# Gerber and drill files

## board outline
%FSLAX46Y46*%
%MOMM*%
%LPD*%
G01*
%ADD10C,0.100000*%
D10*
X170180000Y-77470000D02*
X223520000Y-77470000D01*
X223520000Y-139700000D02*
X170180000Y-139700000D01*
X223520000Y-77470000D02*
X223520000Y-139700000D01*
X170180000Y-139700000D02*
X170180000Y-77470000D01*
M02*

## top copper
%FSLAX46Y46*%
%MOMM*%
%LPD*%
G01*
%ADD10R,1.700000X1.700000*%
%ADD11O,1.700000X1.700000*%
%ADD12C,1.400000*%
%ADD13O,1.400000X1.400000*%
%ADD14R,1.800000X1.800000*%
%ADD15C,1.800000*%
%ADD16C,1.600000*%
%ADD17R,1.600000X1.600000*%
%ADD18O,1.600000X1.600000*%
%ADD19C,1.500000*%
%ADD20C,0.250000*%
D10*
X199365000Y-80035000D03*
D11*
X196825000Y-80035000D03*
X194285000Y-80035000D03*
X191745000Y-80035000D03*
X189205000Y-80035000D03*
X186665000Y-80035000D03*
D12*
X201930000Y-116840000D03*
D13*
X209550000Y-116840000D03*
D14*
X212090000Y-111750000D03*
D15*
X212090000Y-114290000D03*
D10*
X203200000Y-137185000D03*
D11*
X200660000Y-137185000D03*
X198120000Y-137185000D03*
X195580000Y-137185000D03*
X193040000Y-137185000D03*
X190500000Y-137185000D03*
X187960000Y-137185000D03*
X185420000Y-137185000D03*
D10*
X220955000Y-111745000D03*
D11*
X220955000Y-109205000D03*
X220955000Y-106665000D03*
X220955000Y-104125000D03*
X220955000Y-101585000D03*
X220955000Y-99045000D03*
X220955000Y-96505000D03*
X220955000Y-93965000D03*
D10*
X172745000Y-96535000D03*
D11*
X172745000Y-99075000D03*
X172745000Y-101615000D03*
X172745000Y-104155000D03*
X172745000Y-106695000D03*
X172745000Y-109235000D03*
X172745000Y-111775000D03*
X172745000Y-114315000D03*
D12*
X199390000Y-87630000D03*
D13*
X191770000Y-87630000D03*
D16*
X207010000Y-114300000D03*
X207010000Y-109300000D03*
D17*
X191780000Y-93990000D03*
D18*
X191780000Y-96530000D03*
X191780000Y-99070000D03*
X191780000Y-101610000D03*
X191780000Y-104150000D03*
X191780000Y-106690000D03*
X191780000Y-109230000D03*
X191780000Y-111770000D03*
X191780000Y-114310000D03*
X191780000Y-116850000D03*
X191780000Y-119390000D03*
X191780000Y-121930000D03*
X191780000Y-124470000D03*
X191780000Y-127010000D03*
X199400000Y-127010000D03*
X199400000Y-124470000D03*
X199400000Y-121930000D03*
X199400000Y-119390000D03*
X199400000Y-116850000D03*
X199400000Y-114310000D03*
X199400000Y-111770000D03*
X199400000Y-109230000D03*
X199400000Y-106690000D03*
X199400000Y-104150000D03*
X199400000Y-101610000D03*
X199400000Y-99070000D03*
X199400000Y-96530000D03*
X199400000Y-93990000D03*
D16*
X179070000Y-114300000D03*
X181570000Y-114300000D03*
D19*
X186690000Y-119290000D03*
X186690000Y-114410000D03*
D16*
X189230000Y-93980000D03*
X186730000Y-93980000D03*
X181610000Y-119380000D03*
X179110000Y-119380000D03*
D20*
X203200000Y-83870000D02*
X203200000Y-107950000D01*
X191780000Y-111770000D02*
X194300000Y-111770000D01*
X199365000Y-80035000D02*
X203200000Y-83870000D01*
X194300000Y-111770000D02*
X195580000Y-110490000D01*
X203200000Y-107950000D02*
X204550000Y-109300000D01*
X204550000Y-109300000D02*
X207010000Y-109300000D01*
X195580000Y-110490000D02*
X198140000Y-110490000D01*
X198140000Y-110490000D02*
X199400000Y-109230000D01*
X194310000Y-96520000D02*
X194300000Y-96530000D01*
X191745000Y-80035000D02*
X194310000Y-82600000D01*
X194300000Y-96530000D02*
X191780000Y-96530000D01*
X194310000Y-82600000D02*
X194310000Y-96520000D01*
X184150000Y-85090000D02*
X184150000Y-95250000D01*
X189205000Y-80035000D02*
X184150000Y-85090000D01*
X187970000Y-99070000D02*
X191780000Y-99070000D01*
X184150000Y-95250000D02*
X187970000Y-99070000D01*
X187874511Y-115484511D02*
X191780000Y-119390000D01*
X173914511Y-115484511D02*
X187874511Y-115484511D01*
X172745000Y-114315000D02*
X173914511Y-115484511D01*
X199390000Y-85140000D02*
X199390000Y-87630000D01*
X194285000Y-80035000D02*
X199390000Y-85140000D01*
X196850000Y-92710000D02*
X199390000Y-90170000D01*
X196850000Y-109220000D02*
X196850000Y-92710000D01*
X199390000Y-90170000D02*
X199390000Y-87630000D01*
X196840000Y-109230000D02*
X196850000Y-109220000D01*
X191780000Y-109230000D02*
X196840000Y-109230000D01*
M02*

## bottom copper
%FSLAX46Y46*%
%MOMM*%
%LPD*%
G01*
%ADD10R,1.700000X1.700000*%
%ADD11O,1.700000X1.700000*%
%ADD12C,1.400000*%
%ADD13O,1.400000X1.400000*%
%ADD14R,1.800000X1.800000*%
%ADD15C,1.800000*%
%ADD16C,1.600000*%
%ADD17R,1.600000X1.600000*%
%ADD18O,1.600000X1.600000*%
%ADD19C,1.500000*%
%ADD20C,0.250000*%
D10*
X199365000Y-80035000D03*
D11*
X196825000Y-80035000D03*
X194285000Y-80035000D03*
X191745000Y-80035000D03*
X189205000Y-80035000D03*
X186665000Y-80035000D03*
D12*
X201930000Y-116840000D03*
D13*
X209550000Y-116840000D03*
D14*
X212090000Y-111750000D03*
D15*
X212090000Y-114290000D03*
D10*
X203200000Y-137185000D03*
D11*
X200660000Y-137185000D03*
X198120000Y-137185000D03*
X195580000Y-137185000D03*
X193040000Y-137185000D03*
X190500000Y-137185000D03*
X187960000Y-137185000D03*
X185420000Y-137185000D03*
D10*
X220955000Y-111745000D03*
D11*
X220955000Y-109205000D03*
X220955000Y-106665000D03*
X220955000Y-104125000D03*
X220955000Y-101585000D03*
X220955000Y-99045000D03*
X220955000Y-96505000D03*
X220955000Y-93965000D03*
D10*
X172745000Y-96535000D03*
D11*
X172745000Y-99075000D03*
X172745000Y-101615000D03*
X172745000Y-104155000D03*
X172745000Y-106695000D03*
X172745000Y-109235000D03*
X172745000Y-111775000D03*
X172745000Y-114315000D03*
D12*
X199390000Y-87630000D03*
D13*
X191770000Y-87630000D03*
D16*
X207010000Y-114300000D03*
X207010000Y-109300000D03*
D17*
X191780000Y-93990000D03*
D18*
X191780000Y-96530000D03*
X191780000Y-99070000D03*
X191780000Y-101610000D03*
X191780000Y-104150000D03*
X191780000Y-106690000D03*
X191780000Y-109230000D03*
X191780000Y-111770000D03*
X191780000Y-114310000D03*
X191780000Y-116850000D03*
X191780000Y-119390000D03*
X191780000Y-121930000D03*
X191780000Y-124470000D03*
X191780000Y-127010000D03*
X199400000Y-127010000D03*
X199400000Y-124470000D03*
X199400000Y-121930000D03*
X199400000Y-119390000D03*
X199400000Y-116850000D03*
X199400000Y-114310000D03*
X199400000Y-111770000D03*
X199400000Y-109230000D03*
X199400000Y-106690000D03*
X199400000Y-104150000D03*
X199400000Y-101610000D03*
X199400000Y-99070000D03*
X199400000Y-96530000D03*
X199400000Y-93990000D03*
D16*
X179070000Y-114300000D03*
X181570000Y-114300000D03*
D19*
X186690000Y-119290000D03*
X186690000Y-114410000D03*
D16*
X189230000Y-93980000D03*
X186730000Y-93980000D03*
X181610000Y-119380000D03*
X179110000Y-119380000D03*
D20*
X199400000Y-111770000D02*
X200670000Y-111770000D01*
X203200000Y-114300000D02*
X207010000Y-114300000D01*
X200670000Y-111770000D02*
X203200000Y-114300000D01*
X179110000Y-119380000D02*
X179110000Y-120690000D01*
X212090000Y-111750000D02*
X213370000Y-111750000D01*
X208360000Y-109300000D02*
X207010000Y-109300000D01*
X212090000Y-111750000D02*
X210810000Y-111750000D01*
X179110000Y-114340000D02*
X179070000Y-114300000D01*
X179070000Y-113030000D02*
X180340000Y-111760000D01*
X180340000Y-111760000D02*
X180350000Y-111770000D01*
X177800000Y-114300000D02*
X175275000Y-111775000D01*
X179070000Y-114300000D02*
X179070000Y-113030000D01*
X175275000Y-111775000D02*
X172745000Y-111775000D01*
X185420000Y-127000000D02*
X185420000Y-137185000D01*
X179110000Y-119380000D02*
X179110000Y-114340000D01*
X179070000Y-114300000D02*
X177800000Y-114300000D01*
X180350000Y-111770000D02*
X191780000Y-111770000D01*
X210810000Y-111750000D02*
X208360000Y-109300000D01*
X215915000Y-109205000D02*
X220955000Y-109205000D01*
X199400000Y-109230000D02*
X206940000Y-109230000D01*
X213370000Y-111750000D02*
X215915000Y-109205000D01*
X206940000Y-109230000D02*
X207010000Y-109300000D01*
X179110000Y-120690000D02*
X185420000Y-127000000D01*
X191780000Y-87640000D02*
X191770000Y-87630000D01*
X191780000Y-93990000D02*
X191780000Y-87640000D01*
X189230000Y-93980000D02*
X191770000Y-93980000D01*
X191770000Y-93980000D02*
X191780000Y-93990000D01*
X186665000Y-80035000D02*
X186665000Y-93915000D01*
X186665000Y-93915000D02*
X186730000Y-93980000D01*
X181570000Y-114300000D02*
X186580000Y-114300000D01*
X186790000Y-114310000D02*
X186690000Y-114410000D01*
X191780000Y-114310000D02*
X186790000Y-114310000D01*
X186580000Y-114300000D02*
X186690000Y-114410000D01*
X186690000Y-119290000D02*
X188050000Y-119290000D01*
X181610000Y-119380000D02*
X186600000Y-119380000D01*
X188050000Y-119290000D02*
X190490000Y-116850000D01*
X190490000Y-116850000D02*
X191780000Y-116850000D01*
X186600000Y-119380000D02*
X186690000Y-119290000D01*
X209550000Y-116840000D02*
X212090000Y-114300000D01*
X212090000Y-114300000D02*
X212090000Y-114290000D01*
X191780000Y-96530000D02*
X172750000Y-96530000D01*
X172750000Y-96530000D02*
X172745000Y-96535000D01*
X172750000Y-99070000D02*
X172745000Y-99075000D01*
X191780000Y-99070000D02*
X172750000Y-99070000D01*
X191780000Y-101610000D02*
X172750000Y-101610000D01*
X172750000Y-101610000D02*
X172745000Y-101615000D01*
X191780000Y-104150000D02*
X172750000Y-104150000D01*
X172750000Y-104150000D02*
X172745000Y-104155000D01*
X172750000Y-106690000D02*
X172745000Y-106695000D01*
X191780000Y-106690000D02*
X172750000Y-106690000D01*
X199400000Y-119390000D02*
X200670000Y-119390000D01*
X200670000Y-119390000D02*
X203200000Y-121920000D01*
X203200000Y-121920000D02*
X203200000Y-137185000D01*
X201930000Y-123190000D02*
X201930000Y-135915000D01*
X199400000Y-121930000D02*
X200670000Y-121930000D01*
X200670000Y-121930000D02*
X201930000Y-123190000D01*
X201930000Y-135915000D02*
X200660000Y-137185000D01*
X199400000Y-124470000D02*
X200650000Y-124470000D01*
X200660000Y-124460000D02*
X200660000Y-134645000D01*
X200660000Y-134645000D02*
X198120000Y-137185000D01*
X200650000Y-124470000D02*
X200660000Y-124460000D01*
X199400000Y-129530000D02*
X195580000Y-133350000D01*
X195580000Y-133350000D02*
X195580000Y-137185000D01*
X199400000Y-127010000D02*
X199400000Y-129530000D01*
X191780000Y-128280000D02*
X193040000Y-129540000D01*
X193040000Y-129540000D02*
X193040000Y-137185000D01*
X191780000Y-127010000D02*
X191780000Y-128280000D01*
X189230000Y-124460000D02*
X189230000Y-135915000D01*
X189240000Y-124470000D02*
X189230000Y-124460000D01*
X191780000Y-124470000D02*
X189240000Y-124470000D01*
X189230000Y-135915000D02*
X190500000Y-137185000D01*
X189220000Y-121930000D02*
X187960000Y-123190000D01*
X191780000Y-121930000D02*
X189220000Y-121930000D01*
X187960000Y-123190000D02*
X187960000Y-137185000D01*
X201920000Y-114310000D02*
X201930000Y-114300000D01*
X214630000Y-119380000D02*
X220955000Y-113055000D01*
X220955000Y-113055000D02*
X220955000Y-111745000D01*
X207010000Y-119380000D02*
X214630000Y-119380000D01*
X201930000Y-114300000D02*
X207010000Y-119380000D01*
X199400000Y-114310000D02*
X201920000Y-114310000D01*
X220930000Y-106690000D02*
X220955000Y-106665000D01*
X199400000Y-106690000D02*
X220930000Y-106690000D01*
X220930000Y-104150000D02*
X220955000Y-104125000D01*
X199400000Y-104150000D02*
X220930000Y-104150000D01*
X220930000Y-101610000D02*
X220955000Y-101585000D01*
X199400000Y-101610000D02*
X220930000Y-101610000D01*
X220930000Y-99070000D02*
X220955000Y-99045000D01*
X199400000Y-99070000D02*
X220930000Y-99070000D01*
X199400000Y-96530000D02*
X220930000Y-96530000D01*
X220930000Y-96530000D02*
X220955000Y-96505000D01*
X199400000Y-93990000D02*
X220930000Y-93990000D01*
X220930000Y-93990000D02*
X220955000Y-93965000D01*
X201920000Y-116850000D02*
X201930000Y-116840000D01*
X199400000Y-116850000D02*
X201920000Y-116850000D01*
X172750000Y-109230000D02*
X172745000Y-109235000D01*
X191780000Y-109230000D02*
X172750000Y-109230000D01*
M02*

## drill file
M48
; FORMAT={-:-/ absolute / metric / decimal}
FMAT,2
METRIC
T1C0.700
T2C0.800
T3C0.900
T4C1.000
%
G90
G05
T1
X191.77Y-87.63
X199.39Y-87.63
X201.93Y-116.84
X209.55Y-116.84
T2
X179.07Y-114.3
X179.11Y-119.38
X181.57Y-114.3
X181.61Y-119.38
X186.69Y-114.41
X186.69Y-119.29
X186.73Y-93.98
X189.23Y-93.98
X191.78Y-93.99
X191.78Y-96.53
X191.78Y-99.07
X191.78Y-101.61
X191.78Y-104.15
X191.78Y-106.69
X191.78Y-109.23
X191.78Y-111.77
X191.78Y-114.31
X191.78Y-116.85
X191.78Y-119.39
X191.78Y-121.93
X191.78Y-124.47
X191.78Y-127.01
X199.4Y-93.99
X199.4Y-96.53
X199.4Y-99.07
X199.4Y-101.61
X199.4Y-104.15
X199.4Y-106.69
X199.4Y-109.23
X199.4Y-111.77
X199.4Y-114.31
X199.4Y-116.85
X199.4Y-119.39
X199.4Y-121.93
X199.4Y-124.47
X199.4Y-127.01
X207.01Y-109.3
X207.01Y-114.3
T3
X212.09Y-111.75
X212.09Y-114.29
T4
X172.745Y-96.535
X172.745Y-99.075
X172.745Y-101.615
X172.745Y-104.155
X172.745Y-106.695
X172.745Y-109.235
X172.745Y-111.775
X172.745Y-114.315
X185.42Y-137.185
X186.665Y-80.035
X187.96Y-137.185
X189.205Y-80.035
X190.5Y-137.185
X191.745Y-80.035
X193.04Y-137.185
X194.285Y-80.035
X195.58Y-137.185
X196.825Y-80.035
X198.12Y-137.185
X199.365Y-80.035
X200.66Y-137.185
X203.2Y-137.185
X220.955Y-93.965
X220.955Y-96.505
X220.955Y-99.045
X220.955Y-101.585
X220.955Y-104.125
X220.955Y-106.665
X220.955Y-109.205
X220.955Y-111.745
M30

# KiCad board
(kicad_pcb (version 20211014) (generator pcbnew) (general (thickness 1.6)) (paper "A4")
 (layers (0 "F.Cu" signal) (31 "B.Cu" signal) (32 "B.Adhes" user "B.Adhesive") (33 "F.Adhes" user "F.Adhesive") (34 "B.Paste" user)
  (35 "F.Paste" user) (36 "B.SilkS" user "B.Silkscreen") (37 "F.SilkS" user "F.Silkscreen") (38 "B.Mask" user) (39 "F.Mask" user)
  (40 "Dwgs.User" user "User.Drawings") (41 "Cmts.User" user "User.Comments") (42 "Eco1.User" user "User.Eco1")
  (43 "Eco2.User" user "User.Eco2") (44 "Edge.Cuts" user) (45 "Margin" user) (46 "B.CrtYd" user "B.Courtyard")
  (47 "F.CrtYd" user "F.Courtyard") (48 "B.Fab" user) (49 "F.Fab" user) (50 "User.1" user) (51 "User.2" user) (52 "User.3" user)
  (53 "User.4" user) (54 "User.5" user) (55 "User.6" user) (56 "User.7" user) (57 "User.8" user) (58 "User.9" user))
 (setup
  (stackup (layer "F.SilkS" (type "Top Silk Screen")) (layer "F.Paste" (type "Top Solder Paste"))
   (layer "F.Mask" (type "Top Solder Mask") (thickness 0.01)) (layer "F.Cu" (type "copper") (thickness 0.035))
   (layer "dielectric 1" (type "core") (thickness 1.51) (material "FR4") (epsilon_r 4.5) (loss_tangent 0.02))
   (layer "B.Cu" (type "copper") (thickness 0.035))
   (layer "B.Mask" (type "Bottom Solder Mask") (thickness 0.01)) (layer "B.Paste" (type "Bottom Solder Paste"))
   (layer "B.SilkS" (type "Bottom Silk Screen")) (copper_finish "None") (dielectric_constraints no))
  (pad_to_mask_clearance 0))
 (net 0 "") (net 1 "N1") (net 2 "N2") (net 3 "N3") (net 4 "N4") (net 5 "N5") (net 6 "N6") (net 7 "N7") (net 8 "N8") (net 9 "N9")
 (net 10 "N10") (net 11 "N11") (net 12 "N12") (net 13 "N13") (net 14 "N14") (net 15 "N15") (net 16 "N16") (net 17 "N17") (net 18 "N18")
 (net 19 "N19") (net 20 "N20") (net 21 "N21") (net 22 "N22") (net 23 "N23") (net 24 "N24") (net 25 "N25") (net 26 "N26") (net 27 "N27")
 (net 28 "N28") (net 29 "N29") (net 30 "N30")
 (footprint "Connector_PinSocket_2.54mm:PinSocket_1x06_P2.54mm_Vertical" (layer "F.Cu") (at 199.365 80.035 -90)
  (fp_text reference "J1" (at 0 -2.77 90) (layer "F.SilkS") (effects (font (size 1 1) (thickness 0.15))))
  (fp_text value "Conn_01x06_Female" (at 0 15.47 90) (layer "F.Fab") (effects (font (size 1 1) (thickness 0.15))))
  (pad "1" thru_hole rect locked (at 0 0 270) (size 1.7 1.7) (drill 1) (layers *.Cu *.Mask) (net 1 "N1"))
  (pad "2" thru_hole oval locked (at 0 2.54 270) (size 1.7 1.7) (drill 1) (layers *.Cu *.Mask) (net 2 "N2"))
  (pad "3" thru_hole oval locked (at 0 5.08 270) (size 1.7 1.7) (drill 1) (layers *.Cu *.Mask) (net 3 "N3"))
  (pad "4" thru_hole oval locked (at 0 7.62 270) (size 1.7 1.7) (drill 1) (layers *.Cu *.Mask) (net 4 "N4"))
  (pad "5" thru_hole oval locked (at 0 10.16 270) (size 1.7 1.7) (drill 1) (layers *.Cu *.Mask) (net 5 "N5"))
  (pad "6" thru_hole oval locked (at 0 12.7 270) (size 1.7 1.7) (drill 1) (layers *.Cu *.Mask) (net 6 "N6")))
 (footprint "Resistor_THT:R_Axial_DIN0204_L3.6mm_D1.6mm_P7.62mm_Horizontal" (layer "F.Cu") (at 201.93 116.84)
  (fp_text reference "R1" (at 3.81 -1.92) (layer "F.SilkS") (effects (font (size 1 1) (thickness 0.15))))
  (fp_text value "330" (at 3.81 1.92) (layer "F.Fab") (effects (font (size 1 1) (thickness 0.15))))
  (pad "1" thru_hole circle locked (at 0 0) (size 1.4 1.4) (drill 0.7) (layers *.Cu *.Mask) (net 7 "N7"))
  (pad "2" thru_hole oval locked (at 7.62 0) (size 1.4 1.4) (drill 0.7) (layers *.Cu *.Mask) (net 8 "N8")))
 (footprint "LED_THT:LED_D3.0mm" (layer "F.Cu") (at 212.09 111.75 -90)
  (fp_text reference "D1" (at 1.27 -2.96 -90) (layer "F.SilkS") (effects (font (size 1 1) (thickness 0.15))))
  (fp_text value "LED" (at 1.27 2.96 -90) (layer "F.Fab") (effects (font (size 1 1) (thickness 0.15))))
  (pad "1" thru_hole rect locked (at 0 0 270) (size 1.8 1.8) (drill 0.9) (layers *.Cu *.Mask) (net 1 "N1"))
  (pad "2" thru_hole circle locked (at 2.54 0 270) (size 1.8 1.8) (drill 0.9) (layers *.Cu *.Mask) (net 8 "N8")))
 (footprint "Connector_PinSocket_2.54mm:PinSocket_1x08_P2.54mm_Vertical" (layer "F.Cu") (at 203.2 137.185 -90)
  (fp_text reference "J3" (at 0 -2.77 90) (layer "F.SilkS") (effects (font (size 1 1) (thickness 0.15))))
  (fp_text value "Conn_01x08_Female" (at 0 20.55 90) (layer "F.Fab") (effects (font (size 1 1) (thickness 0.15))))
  (pad "1" thru_hole rect locked (at 0 0 270) (size 1.7 1.7) (drill 1) (layers *.Cu *.Mask) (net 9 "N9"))
  (pad "2" thru_hole oval locked (at 0 2.54 270) (size 1.7 1.7) (drill 1) (layers *.Cu *.Mask) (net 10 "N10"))
  (pad "3" thru_hole oval locked (at 0 5.08 270) (size 1.7 1.7) (drill 1) (layers *.Cu *.Mask) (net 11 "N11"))
  (pad "4" thru_hole oval locked (at 0 7.62 270) (size 1.7 1.7) (drill 1) (layers *.Cu *.Mask) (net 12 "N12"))
  (pad "5" thru_hole oval locked (at 0 10.16 270) (size 1.7 1.7) (drill 1) (layers *.Cu *.Mask) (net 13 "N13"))
  (pad "6" thru_hole oval locked (at 0 12.7 270) (size 1.7 1.7) (drill 1) (layers *.Cu *.Mask) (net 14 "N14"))
  (pad "7" thru_hole oval locked (at 0 15.24 270) (size 1.7 1.7) (drill 1) (layers *.Cu *.Mask) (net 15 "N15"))
  (pad "8" thru_hole oval locked (at 0 17.78 270) (size 1.7 1.7) (drill 1) (layers *.Cu *.Mask) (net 1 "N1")))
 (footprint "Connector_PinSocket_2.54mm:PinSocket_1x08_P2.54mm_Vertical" (layer "F.Cu") (at 220.955 111.745 180)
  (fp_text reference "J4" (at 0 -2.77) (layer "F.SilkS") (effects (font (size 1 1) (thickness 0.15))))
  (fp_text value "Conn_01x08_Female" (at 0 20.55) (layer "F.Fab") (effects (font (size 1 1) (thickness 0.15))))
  (pad "1" thru_hole rect locked (at 0 0 180) (size 1.7 1.7) (drill 1) (layers *.Cu *.Mask) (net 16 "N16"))
  (pad "2" thru_hole oval locked (at 0 2.54 180) (size 1.7 1.7) (drill 1) (layers *.Cu *.Mask) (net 1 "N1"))
  (pad "3" thru_hole oval locked (at 0 5.08 180) (size 1.7 1.7) (drill 1) (layers *.Cu *.Mask) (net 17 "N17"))
  (pad "4" thru_hole oval locked (at 0 7.62 180) (size 1.7 1.7) (drill 1) (layers *.Cu *.Mask) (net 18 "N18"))
  (pad "5" thru_hole oval locked (at 0 10.16 180) (size 1.7 1.7) (drill 1) (layers *.Cu *.Mask) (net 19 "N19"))
  (pad "6" thru_hole oval locked (at 0 12.7 180) (size 1.7 1.7) (drill 1) (layers *.Cu *.Mask) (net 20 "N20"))
  (pad "7" thru_hole oval locked (at 0 15.24 180) (size 1.7 1.7) (drill 1) (layers *.Cu *.Mask) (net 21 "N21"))
  (pad "8" thru_hole oval locked (at 0 17.78 180) (size 1.7 1.7) (drill 1) (layers *.Cu *.Mask) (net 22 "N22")))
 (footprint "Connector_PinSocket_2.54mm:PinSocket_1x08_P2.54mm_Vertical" (layer "F.Cu") (at 172.745 96.535)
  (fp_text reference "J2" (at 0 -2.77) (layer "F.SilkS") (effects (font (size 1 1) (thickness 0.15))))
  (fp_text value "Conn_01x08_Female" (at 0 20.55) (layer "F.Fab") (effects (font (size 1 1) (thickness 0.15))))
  (pad "1" thru_hole rect locked (at 0 0) (size 1.7 1.7) (drill 1) (layers *.Cu *.Mask) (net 4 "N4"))
  (pad "2" thru_hole oval locked (at 0 2.54) (size 1.7 1.7) (drill 1) (layers *.Cu *.Mask) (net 5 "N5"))
  (pad "3" thru_hole oval locked (at 0 5.08) (size 1.7 1.7) (drill 1) (layers *.Cu *.Mask) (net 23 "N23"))
  (pad "4" thru_hole oval locked (at 0 7.62) (size 1.7 1.7) (drill 1) (layers *.Cu *.Mask) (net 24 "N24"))
  (pad "5" thru_hole oval locked (at 0 10.16) (size 1.7 1.7) (drill 1) (layers *.Cu *.Mask) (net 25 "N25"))
  (pad "6" thru_hole oval locked (at 0 12.7) (size 1.7 1.7) (drill 1) (layers *.Cu *.Mask) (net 3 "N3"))
  (pad "7" thru_hole oval locked (at 0 15.24) (size 1.7 1.7) (drill 1) (layers *.Cu *.Mask) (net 1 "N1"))
  (pad "8" thru_hole oval locked (at 0 17.78) (size 1.7 1.7) (drill 1) (layers *.Cu *.Mask) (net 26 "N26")))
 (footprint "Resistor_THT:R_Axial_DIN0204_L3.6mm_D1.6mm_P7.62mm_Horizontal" (layer "F.Cu") (at 199.39 87.63 180)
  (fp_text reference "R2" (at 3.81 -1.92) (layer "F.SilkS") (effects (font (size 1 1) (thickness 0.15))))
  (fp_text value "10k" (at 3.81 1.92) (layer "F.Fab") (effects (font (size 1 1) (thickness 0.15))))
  (pad "1" thru_hole circle locked (at 0 0 180) (size 1.4 1.4) (drill 0.7) (layers *.Cu *.Mask) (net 3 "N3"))
  (pad "2" thru_hole oval locked (at 7.62 0 180) (size 1.4 1.4) (drill 0.7) (layers *.Cu *.Mask) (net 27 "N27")))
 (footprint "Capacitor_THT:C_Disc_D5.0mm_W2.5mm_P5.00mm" (layer "F.Cu") (at 207.01 114.3 90)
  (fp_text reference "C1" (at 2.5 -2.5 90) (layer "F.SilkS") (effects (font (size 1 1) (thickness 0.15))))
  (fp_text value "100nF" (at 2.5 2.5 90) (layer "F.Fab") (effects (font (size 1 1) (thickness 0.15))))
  (pad "1" thru_hole circle locked (at 0 0 90) (size 1.6 1.6) (drill 0.8) (layers *.Cu *.Mask) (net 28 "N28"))
  (pad "2" thru_hole circle locked (at 5 0 90) (size 1.6 1.6) (drill 0.8) (layers *.Cu *.Mask) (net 1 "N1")))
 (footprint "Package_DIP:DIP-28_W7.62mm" (layer "F.Cu") (at 191.78 93.99)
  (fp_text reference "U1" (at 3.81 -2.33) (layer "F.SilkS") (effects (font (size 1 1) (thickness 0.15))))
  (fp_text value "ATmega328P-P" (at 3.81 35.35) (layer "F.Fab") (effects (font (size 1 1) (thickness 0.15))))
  (pad "1" thru_hole rect locked (at 0 0) (size 1.6 1.6) (drill 0.8) (layers *.Cu *.Mask) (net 27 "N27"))
  (pad "2" thru_hole oval locked (at 0 2.54) (size 1.6 1.6) (drill 0.8) (layers *.Cu *.Mask) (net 4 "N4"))
  (pad "3" thru_hole oval locked (at 0 5.08) (size 1.6 1.6) (drill 0.8) (layers *.Cu *.Mask) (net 5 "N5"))
  (pad "4" thru_hole oval locked (at 0 7.62) (size 1.6 1.6) (drill 0.8) (layers *.Cu *.Mask) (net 23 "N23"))
  (pad "5" thru_hole oval locked (at 0 10.16) (size 1.6 1.6) (drill 0.8) (layers *.Cu *.Mask) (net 24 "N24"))
  (pad "6" thru_hole oval locked (at 0 12.7) (size 1.6 1.6) (drill 0.8) (layers *.Cu *.Mask) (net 25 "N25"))
  (pad "7" thru_hole oval locked (at 0 15.24) (size 1.6 1.6) (drill 0.8) (layers *.Cu *.Mask) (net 3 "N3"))
  (pad "8" thru_hole oval locked (at 0 17.78) (size 1.6 1.6) (drill 0.8) (layers *.Cu *.Mask) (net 1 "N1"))
  (pad "9" thru_hole oval locked (at 0 20.32) (size 1.6 1.6) (drill 0.8) (layers *.Cu *.Mask) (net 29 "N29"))
  (pad "10" thru_hole oval locked (at 0 22.86) (size 1.6 1.6) (drill 0.8) (layers *.Cu *.Mask) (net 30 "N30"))
  (pad "11" thru_hole oval locked (at 0 25.4) (size 1.6 1.6) (drill 0.8) (layers *.Cu *.Mask) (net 26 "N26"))
  (pad "12" thru_hole oval locked (at 0 27.94) (size 1.6 1.6) (drill 0.8) (layers *.Cu *.Mask) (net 15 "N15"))
  (pad "13" thru_hole oval locked (at 0 30.48) (size 1.6 1.6) (drill 0.8) (layers *.Cu *.Mask) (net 14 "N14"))
  (pad "14" thru_hole oval locked (at 0 33.02) (size 1.6 1.6) (drill 0.8) (layers *.Cu *.Mask) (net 13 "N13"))
  (pad "15" thru_hole oval locked (at 7.62 33.02) (size 1.6 1.6) (drill 0.8) (layers *.Cu *.Mask) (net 12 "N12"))
  (pad "16" thru_hole oval locked (at 7.62 30.48) (size 1.6 1.6) (drill 0.8) (layers *.Cu *.Mask) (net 11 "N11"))
  (pad "17" thru_hole oval locked (at 7.62 27.94) (size 1.6 1.6) (drill 0.8) (layers *.Cu *.Mask) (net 10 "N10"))
  (pad "18" thru_hole oval locked (at 7.62 25.4) (size 1.6 1.6) (drill 0.8) (layers *.Cu *.Mask) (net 9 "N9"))
  (pad "19" thru_hole oval locked (at 7.62 22.86) (size 1.6 1.6) (drill 0.8) (layers *.Cu *.Mask) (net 7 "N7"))
  (pad "20" thru_hole oval locked (at 7.62 20.32) (size 1.6 1.6) (drill 0.8) (layers *.Cu *.Mask) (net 16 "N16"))
  (pad "21" thru_hole oval locked (at 7.62 17.78) (size 1.6 1.6) (drill 0.8) (layers *.Cu *.Mask) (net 28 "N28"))
  (pad "22" thru_hole oval locked (at 7.62 15.24) (size 1.6 1.6) (drill 0.8) (layers *.Cu *.Mask) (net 1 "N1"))
  (pad "23" thru_hole oval locked (at 7.62 12.7) (size 1.6 1.6) (drill 0.8) (layers *.Cu *.Mask) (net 17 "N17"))
  (pad "24" thru_hole oval locked (at 7.62 10.16) (size 1.6 1.6) (drill 0.8) (layers *.Cu *.Mask) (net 18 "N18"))
  (pad "25" thru_hole oval locked (at 7.62 7.62) (size 1.6 1.6) (drill 0.8) (layers *.Cu *.Mask) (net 19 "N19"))
  (pad "26" thru_hole oval locked (at 7.62 5.08) (size 1.6 1.6) (drill 0.8) (layers *.Cu *.Mask) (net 20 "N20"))
  (pad "27" thru_hole oval locked (at 7.62 2.54) (size 1.6 1.6) (drill 0.8) (layers *.Cu *.Mask) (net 21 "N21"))
  (pad "28" thru_hole oval locked (at 7.62 0) (size 1.6 1.6) (drill 0.8) (layers *.Cu *.Mask) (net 22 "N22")))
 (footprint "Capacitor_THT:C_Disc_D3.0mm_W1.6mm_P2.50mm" (layer "F.Cu") (at 179.07 114.3)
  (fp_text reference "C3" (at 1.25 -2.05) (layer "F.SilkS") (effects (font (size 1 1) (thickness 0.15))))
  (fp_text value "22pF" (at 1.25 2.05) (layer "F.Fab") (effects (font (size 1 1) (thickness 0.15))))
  (pad "1" thru_hole circle locked (at 0 0) (size 1.6 1.6) (drill 0.8) (layers *.Cu *.Mask) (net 1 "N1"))
  (pad "2" thru_hole circle locked (at 2.5 0) (size 1.6 1.6) (drill 0.8) (layers *.Cu *.Mask) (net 29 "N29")))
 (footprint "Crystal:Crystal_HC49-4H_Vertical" (layer "F.Cu") (at 186.69 119.29 90)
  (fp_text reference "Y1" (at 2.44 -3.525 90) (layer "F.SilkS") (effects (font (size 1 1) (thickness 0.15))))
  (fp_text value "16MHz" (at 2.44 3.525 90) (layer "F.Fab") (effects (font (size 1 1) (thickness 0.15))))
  (pad "1" thru_hole circle locked (at 0 0 90) (size 1.5 1.5) (drill 0.8) (layers *.Cu *.Mask) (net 30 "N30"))
  (pad "2" thru_hole circle locked (at 4.88 0 90) (size 1.5 1.5) (drill 0.8) (layers *.Cu *.Mask) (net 29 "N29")))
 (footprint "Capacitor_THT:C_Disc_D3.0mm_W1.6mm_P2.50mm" (layer "F.Cu") (at 189.23 93.98 180)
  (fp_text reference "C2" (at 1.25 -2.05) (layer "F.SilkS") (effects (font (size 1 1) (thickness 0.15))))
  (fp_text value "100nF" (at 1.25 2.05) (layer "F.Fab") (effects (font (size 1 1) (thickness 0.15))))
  (pad "1" thru_hole circle locked (at 0 0 180) (size 1.6 1.6) (drill 0.8) (layers *.Cu *.Mask) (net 27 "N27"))
  (pad "2" thru_hole circle locked (at 2.5 0 180) (size 1.6 1.6) (drill 0.8) (layers *.Cu *.Mask) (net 6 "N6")))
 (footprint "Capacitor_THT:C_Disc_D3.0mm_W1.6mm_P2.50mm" (layer "F.Cu") (at 181.61 119.38 180)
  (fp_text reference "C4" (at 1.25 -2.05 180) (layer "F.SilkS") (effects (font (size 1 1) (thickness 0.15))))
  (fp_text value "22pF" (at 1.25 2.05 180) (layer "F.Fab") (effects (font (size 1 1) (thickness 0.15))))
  (pad "1" thru_hole circle locked (at 0 0 180) (size 1.6 1.6) (drill 0.8) (layers *.Cu *.Mask) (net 30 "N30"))
  (pad "2" thru_hole circle locked (at 2.5 0 180) (size 1.6 1.6) (drill 0.8) (layers *.Cu *.Mask) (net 1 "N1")))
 (gr_line (start 170.18 77.47) (end 223.52 77.47) (layer "Edge.Cuts") (width 0.1))
 (gr_line (start 223.52 139.7) (end 170.18 139.7) (layer "Edge.Cuts") (width 0.1))
 (gr_line (start 223.52 77.47) (end 223.52 139.7) (layer "Edge.Cuts") (width 0.1))
 (gr_line (start 170.18 139.7) (end 170.18 77.47) (layer "Edge.Cuts") (width 0.1))
 (segment (start 199.4 111.77) (end 200.67 111.77) (width 0.25) (layer "B.Cu") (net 28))
 (segment (start 203.2 114.3) (end 207.01 114.3) (width 0.25) (layer "B.Cu") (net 28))
 (segment (start 200.67 111.77) (end 203.2 114.3) (width 0.25) (layer "B.Cu") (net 28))
 (segment (start 203.2 83.87) (end 203.2 107.95) (width 0.25) (layer "F.Cu") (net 1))
 (segment (start 191.78 111.77) (end 194.3 111.77) (width 0.25) (layer "F.Cu") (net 1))
 (segment (start 199.365 80.035) (end 203.2 83.87) (width 0.25) (layer "F.Cu") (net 1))
 (segment (start 194.3 111.77) (end 195.58 110.49) (width 0.25) (layer "F.Cu") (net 1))
 (segment (start 203.2 107.95) (end 204.55 109.3) (width 0.25) (layer "F.Cu") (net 1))
 (segment (start 204.55 109.3) (end 207.01 109.3) (width 0.25) (layer "F.Cu") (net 1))
 (segment (start 195.58 110.49) (end 198.14 110.49) (width 0.25) (layer "F.Cu") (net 1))
 (segment (start 198.14 110.49) (end 199.4 109.23) (width 0.25) (layer "F.Cu") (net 1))
 (segment (start 179.11 119.38) (end 179.11 120.69) (width 0.25) (layer "B.Cu") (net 1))
 (segment (start 212.09 111.75) (end 213.37 111.75) (width 0.25) (layer "B.Cu") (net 1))
 (segment (start 208.36 109.3) (end 207.01 109.3) (width 0.25) (layer "B.Cu") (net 1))
 (segment (start 212.09 111.75) (end 210.81 111.75) (width 0.25) (layer "B.Cu") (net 1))
 (segment (start 179.11 114.34) (end 179.07 114.3) (width 0.25) (layer "B.Cu") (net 1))
 (segment (start 179.07 113.03) (end 180.34 111.76) (width 0.25) (layer "B.Cu") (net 1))
 (segment (start 180.34 111.76) (end 180.35 111.77) (width 0.25) (layer "B.Cu") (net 1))
 (segment (start 177.8 114.3) (end 175.275 111.775) (width 0.25) (layer "B.Cu") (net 1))
 (segment (start 179.07 114.3) (end 179.07 113.03) (width 0.25) (layer "B.Cu") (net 1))
 (segment (start 175.275 111.775) (end 172.745 111.775) (width 0.25) (layer "B.Cu") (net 1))
 (segment (start 185.42 127) (end 185.42 137.185) (width 0.25) (layer "B.Cu") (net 1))
 (segment (start 179.11 119.38) (end 179.11 114.34) (width 0.25) (layer "B.Cu") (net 1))
 (segment (start 179.07 114.3) (end 177.8 114.3) (width 0.25) (layer "B.Cu") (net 1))
 (segment (start 180.35 111.77) (end 191.78 111.77) (width 0.25) (layer "B.Cu") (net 1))
 (segment (start 210.81 111.75) (end 208.36 109.3) (width 0.25) (layer "B.Cu") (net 1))
 (segment (start 215.915 109.205) (end 220.955 109.205) (width 0.25) (layer "B.Cu") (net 1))
 (segment (start 199.4 109.23) (end 206.94 109.23) (width 0.25) (layer "B.Cu") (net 1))
 (segment (start 213.37 111.75) (end 215.915 109.205) (width 0.25) (layer "B.Cu") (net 1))
 (segment (start 206.94 109.23) (end 207.01 109.3) (width 0.25) (layer "B.Cu") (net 1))
 (segment (start 179.11 120.69) (end 185.42 127) (width 0.25) (layer "B.Cu") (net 1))
 (segment (start 191.78 87.64) (end 191.77 87.63) (width 0.25) (layer "B.Cu") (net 27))
 (segment (start 191.78 93.99) (end 191.78 87.64) (width 0.25) (layer "B.Cu") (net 27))
 (segment (start 189.23 93.98) (end 191.77 93.98) (width 0.25) (layer "B.Cu") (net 27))
 (segment (start 191.77 93.98) (end 191.78 93.99) (width 0.25) (layer "B.Cu") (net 27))
 (segment (start 186.665 80.035) (end 186.665 93.915) (width 0.25) (layer "B.Cu") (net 6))
 (segment (start 186.665 93.915) (end 186.73 93.98) (width 0.25) (layer "B.Cu") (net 6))
 (segment (start 181.57 114.3) (end 186.58 114.3) (width 0.25) (layer "B.Cu") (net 29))
 (segment (start 186.79 114.31) (end 186.69 114.41) (width 0.25) (layer "B.Cu") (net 29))
 (segment (start 191.78 114.31) (end 186.79 114.31) (width 0.25) (layer "B.Cu") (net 29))
 (segment (start 186.58 114.3) (end 186.69 114.41) (width 0.25) (layer "B.Cu") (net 29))
 (segment (start 186.69 119.29) (end 188.05 119.29) (width 0.25) (layer "B.Cu") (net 30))
 (segment (start 181.61 119.38) (end 186.6 119.38) (width 0.25) (layer "B.Cu") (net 30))
 (segment (start 188.05 119.29) (end 190.49 116.85) (width 0.25) (layer "B.Cu") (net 30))
 (segment (start 190.49 116.85) (end 191.78 116.85) (width 0.25) (layer "B.Cu") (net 30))
 (segment (start 186.6 119.38) (end 186.69 119.29) (width 0.25) (layer "B.Cu") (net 30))
 (segment (start 209.55 116.84) (end 212.09 114.3) (width 0.25) (layer "B.Cu") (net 8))
 (segment (start 212.09 114.3) (end 212.09 114.29) (width 0.25) (layer "B.Cu") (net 8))
 (segment (start 194.31 96.52) (end 194.3 96.53) (width 0.25) (layer "F.Cu") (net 4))
 (segment (start 191.745 80.035) (end 194.31 82.6) (width 0.25) (layer "F.Cu") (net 4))
 (segment (start 194.3 96.53) (end 191.78 96.53) (width 0.25) (layer "F.Cu") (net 4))
 (segment (start 194.31 82.6) (end 194.31 96.52) (width 0.25) (layer "F.Cu") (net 4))
 (segment (start 191.78 96.53) (end 172.75 96.53) (width 0.25) (layer "B.Cu") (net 4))
 (segment (start 172.75 96.53) (end 172.745 96.535) (width 0.25) (layer "B.Cu") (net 4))
 (segment (start 184.15 85.09) (end 184.15 95.25) (width 0.25) (layer "F.Cu") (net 5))
 (segment (start 189.205 80.035) (end 184.15 85.09) (width 0.25) (layer "F.Cu") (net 5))
 (segment (start 187.97 99.07) (end 191.78 99.07) (width 0.25) (layer "F.Cu") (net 5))
 (segment (start 184.15 95.25) (end 187.97 99.07) (width 0.25) (layer "F.Cu") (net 5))
 (segment (start 172.75 99.07) (end 172.745 99.075) (width 0.25) (layer "B.Cu") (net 5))
 (segment (start 191.78 99.07) (end 172.75 99.07) (width 0.25) (layer "B.Cu") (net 5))
 (segment (start 191.78 101.61) (end 172.75 101.61) (width 0.25) (layer "B.Cu") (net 23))
 (segment (start 172.75 101.61) (end 172.745 101.615) (width 0.25) (layer "B.Cu") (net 23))
 (segment (start 191.78 104.15) (end 172.75 104.15) (width 0.25) (layer "B.Cu") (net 24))
 (segment (start 172.75 104.15) (end 172.745 104.155) (width 0.25) (layer "B.Cu") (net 24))
 (segment (start 172.75 106.69) (end 172.745 106.695) (width 0.25) (layer "B.Cu") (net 25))
 (segment (start 191.78 106.69) (end 172.75 106.69) (width 0.25) (layer "B.Cu") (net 25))
 (segment (start 187.874511 115.484511) (end 191.78 119.39) (width 0.25) (layer "F.Cu") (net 26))
 (segment (start 173.914511 115.484511) (end 187.874511 115.484511) (width 0.25) (layer "F.Cu") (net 26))
 (segment (start 172.745 114.315) (end 173.914511 115.484511) (width 0.25) (layer "F.Cu") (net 26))
 (segment (start 199.4 119.39) (end 200.67 119.39) (width 0.25) (layer "B.Cu") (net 9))
 (segment (start 200.67 119.39) (end 203.2 121.92) (width 0.25) (layer "B.Cu") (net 9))
 (segment (start 203.2 121.92) (end 203.2 137.185) (width 0.25) (layer "B.Cu") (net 9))
 (segment (start 201.93 123.19) (end 201.93 135.915) (width 0.25) (layer "B.Cu") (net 10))
 (segment (start 199.4 121.93) (end 200.67 121.93) (width 0.25) (layer "B.Cu") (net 10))
 (segment (start 200.67 121.93) (end 201.93 123.19) (width 0.25) (layer "B.Cu") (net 10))
 (segment (start 201.93 135.915) (end 200.66 137.185) (width 0.25) (layer "B.Cu") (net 10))
 (segment (start 199.4 124.47) (end 200.65 124.47) (width 0.25) (layer "B.Cu") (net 11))
 (segment (start 200.66 124.46) (end 200.66 134.645) (width 0.25) (layer "B.Cu") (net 11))
 (segment (start 200.66 134.645) (end 198.12 137.185) (width 0.25) (layer "B.Cu") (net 11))
 (segment (start 200.65 124.47) (end 200.66 124.46) (width 0.25) (layer "B.Cu") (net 11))
 (segment (start 199.4 129.53) (end 195.58 133.35) (width 0.25) (layer "B.Cu") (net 12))
 (segment (start 195.58 133.35) (end 195.58 137.185) (width 0.25) (layer "B.Cu") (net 12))
 (segment (start 199.4 127.01) (end 199.4 129.53) (width 0.25) (layer "B.Cu") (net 12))
 (segment (start 191.78 128.28) (end 193.04 129.54) (width 0.25) (layer "B.Cu") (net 13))
 (segment (start 193.04 129.54) (end 193.04 137.185) (width 0.25) (layer "B.Cu") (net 13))
 (segment (start 191.78 127.01) (end 191.78 128.28) (width 0.25) (layer "B.Cu") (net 13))
 (segment (start 189.23 124.46) (end 189.23 135.915) (width 0.25) (layer "B.Cu") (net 14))
 (segment (start 189.24 124.47) (end 189.23 124.46) (width 0.25) (layer "B.Cu") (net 14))
 (segment (start 191.78 124.47) (end 189.24 124.47) (width 0.25) (layer "B.Cu") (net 14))
 (segment (start 189.23 135.915) (end 190.5 137.185) (width 0.25) (layer "B.Cu") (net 14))
 (segment (start 189.22 121.93) (end 187.96 123.19) (width 0.25) (layer "B.Cu") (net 15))
 (segment (start 191.78 121.93) (end 189.22 121.93) (width 0.25) (layer "B.Cu") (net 15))
 (segment (start 187.96 123.19) (end 187.96 137.185) (width 0.25) (layer "B.Cu") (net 15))
 (segment (start 201.92 114.31) (end 201.93 114.3) (width 0.25) (layer "B.Cu") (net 16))
 (segment (start 214.63 119.38) (end 220.955 113.055) (width 0.25) (layer "B.Cu") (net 16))
 (segment (start 220.955 113.055) (end 220.955 111.745) (width 0.25) (layer "B.Cu") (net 16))
 (segment (start 207.01 119.38) (end 214.63 119.38) (width 0.25) (layer "B.Cu") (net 16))
 (segment (start 201.93 114.3) (end 207.01 119.38) (width 0.25) (layer "B.Cu") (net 16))
 (segment (start 199.4 114.31) (end 201.92 114.31) (width 0.25) (layer "B.Cu") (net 16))
 (segment (start 220.93 106.69) (end 220.955 106.665) (width 0.25) (layer "B.Cu") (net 17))
 (segment (start 199.4 106.69) (end 220.93 106.69) (width 0.25) (layer "B.Cu") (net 17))
 (segment (start 220.93 104.15) (end 220.955 104.125) (width 0.25) (layer "B.Cu") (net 18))
 (segment (start 199.4 104.15) (end 220.93 104.15) (width 0.25) (layer "B.Cu") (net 18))
 (segment (start 220.93 101.61) (end 220.955 101.585) (width 0.25) (layer "B.Cu") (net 19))
 (segment (start 199.4 101.61) (end 220.93 101.61) (width 0.25) (layer "B.Cu") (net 19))
 (segment (start 220.93 99.07) (end 220.955 99.045) (width 0.25) (layer "B.Cu") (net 20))
 (segment (start 199.4 99.07) (end 220.93 99.07) (width 0.25) (layer "B.Cu") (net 20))
 (segment (start 199.4 96.53) (end 220.93 96.53) (width 0.25) (layer "B.Cu") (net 21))
 (segment (start 220.93 96.53) (end 220.955 96.505) (width 0.25) (layer "B.Cu") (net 21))
 (segment (start 199.4 93.99) (end 220.93 93.99) (width 0.25) (layer "B.Cu") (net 22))
 (segment (start 220.93 93.99) (end 220.955 93.965) (width 0.25) (layer "B.Cu") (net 22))
 (segment (start 201.92 116.85) (end 201.93 116.84) (width 0.25) (layer "B.Cu") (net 7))
 (segment (start 199.4 116.85) (end 201.92 116.85) (width 0.25) (layer "B.Cu") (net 7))
 (segment (start 199.39 85.14) (end 199.39 87.63) (width 0.25) (layer "F.Cu") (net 3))
 (segment (start 194.285 80.035) (end 199.39 85.14) (width 0.25) (layer "F.Cu") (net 3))
 (segment (start 196.85 92.71) (end 199.39 90.17) (width 0.25) (layer "F.Cu") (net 3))
 (segment (start 196.85 109.22) (end 196.85 92.71) (width 0.25) (layer "F.Cu") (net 3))
 (segment (start 199.39 90.17) (end 199.39 87.63) (width 0.25) (layer "F.Cu") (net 3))
 (segment (start 196.84 109.23) (end 196.85 109.22) (width 0.25) (layer "F.Cu") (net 3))
 (segment (start 191.78 109.23) (end 196.84 109.23) (width 0.25) (layer "F.Cu") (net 3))
 (segment (start 172.75 109.23) (end 172.745 109.235) (width 0.25) (layer "B.Cu") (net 3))
 (segment (start 191.78 109.23) (end 172.75 109.23) (width 0.25) (layer "B.Cu") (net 3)))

